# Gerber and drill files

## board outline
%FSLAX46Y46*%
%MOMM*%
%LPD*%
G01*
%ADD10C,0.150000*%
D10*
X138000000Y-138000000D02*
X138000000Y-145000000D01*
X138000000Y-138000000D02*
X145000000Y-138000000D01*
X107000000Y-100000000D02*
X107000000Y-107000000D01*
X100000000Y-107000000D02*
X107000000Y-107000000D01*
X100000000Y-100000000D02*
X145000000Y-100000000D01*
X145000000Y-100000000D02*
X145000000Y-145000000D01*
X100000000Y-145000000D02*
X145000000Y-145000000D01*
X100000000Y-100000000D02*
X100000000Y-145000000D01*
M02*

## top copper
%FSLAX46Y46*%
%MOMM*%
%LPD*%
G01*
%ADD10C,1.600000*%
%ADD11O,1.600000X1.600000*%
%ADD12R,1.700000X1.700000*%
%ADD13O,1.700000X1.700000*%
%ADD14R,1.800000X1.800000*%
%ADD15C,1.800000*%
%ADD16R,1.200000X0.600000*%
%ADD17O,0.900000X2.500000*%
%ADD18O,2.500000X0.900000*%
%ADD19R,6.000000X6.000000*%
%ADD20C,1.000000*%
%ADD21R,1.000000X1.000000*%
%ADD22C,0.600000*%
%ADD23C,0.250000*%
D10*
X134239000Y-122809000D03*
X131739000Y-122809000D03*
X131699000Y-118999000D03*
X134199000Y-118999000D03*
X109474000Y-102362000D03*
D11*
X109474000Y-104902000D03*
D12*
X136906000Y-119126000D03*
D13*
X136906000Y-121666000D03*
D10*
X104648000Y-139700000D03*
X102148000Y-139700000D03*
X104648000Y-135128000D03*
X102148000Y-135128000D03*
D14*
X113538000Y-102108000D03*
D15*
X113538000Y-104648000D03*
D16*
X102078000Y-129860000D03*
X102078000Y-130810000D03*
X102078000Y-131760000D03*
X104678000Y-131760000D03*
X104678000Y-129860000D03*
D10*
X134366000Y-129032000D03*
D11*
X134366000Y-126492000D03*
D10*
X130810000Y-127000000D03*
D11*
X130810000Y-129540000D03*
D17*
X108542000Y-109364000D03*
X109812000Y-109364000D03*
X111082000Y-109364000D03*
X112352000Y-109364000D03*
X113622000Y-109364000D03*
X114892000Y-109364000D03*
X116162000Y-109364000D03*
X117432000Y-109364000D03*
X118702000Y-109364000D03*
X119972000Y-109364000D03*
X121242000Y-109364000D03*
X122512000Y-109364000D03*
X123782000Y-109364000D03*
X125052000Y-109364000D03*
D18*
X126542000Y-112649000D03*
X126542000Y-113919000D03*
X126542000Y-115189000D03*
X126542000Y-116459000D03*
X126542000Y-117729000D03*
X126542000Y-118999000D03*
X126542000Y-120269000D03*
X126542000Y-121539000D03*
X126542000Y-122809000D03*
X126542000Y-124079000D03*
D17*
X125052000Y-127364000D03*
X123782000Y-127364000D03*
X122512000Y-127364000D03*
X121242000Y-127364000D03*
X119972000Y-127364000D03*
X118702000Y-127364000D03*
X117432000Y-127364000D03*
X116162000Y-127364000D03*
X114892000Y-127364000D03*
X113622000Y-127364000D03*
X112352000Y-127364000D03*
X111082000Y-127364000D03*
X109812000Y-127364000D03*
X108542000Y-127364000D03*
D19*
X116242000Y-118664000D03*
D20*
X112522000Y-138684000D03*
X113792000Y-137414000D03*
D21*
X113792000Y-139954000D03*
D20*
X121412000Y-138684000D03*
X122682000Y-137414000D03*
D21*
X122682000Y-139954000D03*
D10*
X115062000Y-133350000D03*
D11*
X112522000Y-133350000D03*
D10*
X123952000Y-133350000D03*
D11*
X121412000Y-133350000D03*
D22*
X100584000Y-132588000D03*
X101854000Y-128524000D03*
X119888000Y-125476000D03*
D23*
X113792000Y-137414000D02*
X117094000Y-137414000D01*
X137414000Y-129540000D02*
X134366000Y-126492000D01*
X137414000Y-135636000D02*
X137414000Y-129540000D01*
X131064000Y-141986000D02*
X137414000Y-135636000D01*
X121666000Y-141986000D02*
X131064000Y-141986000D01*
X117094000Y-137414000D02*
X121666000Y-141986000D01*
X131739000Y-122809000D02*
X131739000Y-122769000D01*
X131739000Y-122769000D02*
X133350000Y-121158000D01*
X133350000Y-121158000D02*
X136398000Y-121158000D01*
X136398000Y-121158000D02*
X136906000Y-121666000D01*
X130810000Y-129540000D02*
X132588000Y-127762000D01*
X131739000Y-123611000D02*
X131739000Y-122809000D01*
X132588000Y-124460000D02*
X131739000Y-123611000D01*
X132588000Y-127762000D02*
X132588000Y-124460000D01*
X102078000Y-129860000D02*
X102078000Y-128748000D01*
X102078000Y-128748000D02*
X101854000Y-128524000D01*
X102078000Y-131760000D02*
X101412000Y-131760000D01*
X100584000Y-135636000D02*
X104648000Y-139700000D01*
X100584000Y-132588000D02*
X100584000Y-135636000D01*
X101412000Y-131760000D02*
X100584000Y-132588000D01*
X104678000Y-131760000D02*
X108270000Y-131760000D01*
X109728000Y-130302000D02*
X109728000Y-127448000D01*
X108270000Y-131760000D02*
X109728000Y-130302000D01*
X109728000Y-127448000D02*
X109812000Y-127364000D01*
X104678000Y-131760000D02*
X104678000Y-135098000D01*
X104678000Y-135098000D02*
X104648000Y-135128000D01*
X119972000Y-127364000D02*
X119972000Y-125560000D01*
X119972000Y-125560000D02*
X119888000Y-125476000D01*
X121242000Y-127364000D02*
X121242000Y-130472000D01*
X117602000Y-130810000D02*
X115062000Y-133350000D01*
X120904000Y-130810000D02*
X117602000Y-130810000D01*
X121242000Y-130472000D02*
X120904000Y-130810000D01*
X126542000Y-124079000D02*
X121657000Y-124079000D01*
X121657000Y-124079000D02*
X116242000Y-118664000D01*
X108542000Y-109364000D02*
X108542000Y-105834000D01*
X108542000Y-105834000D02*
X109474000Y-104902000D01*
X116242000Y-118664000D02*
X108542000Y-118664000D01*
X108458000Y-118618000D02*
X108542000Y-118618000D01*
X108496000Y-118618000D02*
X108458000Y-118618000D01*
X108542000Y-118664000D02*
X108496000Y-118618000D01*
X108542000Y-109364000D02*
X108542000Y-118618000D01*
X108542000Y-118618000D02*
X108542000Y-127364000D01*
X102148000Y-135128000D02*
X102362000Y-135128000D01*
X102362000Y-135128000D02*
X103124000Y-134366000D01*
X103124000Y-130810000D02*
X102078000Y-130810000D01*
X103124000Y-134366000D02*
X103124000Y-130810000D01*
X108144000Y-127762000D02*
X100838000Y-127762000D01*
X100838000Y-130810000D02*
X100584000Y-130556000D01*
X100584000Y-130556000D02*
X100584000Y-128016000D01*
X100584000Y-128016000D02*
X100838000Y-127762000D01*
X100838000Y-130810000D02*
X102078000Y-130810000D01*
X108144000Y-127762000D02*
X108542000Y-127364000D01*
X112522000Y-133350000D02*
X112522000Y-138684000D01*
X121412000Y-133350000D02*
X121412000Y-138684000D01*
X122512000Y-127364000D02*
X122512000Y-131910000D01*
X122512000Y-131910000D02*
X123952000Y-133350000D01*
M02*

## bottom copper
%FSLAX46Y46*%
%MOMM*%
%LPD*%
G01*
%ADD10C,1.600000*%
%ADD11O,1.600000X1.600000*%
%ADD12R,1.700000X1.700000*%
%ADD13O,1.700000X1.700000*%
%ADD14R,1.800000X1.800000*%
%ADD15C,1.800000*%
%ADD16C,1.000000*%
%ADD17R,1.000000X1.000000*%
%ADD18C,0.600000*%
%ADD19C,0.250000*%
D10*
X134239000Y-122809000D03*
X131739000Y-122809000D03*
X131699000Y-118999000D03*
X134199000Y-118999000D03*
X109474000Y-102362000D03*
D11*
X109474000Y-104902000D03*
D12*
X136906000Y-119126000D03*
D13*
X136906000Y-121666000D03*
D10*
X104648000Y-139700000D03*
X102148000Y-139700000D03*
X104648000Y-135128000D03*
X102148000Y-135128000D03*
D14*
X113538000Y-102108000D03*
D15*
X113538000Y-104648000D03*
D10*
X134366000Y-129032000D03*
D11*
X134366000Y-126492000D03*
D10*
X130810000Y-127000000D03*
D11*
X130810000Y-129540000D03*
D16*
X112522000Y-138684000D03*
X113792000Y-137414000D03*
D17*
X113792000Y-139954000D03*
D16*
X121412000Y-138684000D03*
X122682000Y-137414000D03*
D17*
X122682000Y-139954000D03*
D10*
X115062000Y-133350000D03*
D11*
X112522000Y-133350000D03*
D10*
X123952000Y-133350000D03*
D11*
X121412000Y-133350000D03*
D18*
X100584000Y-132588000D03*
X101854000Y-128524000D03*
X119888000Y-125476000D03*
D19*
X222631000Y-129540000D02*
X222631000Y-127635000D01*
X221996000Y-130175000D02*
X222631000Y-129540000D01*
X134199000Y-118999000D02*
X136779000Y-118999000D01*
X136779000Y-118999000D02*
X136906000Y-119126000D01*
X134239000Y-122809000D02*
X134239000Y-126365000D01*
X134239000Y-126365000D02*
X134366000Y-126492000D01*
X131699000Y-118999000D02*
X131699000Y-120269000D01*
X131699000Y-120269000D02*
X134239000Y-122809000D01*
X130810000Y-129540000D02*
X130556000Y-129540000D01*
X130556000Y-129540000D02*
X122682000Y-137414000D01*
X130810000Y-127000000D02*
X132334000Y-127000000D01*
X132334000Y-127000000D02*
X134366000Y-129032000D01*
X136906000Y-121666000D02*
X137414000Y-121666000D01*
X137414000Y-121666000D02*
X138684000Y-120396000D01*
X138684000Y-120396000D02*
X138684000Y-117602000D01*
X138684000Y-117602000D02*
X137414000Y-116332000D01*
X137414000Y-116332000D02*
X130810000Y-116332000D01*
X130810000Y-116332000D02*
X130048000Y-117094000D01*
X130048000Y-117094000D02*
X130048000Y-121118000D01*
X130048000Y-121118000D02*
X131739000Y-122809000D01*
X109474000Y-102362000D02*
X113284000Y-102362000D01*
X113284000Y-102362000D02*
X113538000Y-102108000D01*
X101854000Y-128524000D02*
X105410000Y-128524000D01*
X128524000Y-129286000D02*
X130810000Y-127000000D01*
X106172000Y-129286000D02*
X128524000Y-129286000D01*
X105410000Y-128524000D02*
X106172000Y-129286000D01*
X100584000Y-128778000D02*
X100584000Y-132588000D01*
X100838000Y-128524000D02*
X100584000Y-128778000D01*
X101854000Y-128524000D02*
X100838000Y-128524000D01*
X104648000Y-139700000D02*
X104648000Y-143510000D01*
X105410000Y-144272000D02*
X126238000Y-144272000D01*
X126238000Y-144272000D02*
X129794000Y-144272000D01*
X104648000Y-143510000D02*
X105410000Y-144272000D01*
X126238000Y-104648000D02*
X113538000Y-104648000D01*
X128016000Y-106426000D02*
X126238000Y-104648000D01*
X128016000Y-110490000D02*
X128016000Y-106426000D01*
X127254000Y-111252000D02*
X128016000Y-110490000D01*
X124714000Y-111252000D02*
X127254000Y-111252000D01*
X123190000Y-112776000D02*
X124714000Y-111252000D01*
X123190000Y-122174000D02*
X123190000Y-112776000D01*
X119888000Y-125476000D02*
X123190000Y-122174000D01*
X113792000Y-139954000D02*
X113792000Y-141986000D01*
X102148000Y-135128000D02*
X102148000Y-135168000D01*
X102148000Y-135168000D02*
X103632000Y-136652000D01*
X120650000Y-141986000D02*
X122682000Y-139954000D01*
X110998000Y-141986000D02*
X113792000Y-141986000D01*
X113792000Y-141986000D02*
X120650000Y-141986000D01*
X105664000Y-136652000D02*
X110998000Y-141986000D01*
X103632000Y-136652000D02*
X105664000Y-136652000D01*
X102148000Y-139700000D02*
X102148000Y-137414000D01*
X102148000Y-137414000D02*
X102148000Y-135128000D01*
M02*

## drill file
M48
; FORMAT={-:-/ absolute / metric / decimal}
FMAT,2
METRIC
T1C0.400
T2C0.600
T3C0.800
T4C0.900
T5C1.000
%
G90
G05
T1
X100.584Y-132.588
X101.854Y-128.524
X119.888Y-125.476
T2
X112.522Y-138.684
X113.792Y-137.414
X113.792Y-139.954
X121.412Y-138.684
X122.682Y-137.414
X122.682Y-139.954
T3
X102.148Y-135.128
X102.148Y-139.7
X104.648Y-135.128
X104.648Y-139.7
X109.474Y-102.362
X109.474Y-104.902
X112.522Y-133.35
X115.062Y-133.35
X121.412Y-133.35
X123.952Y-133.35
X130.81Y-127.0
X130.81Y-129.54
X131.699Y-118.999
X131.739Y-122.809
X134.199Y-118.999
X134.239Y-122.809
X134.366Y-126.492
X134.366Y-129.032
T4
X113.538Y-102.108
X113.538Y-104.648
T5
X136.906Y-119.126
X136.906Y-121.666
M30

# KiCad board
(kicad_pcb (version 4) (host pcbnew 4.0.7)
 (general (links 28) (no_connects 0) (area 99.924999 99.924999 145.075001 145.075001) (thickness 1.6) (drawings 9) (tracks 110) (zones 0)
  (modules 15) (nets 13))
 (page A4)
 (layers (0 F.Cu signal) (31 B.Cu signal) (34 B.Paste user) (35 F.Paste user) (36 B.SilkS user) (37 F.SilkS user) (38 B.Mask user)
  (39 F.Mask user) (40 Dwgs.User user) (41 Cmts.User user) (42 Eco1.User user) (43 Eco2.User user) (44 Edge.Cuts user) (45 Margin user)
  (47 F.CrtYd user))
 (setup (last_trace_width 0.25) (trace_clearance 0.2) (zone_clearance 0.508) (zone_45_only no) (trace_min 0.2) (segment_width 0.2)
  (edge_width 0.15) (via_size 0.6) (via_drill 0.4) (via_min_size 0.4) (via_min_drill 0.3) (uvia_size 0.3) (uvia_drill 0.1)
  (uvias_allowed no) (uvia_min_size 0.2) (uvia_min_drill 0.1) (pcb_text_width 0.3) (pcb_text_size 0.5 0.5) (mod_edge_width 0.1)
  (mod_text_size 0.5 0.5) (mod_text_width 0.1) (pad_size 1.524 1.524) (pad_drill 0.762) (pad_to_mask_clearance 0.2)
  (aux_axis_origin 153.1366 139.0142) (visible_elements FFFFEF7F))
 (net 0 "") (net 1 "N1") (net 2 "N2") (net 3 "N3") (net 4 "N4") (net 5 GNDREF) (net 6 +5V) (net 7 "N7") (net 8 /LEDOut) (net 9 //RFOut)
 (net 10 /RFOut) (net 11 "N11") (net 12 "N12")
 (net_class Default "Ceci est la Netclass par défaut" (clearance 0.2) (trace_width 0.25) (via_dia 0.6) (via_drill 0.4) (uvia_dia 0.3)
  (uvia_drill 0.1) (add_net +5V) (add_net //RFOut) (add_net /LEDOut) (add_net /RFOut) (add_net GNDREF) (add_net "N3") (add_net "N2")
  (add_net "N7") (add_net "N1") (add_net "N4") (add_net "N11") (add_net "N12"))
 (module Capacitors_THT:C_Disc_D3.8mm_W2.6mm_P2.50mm (layer F.Cu) (at 134.239 122.809 180)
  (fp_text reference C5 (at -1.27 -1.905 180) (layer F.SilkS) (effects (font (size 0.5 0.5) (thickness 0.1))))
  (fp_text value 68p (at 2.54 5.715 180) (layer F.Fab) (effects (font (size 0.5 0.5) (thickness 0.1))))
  (pad 1 thru_hole circle (at 0 0 180) (size 1.6 1.6) (drill 0.8) (layers *.Cu *.Mask) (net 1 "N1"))
  (pad 2 thru_hole circle (at 2.5 0 180) (size 1.6 1.6) (drill 0.8) (layers *.Cu *.Mask) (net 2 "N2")))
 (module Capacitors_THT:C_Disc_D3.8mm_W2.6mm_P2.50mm (layer F.Cu) (at 131.699 118.999)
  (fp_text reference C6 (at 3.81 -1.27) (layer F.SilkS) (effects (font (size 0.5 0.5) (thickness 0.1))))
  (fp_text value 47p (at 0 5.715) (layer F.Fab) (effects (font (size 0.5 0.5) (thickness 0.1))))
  (pad 1 thru_hole circle (at 0 0) (size 1.6 1.6) (drill 0.8) (layers *.Cu *.Mask) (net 1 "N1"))
  (pad 2 thru_hole circle (at 2.5 0) (size 1.6 1.6) (drill 0.8) (layers *.Cu *.Mask) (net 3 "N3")))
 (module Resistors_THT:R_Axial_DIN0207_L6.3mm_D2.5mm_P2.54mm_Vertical (layer F.Cu) (at 109.474 102.362 270)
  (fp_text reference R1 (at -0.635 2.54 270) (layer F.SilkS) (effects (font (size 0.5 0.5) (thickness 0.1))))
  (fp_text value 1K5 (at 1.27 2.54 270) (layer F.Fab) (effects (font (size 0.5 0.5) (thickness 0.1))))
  (pad 1 thru_hole circle (at 0 0 270) (size 1.6 1.6) (drill 0.8) (layers *.Cu *.Mask) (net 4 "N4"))
  (pad 2 thru_hole oval (at 2.54 0 270) (size 1.6 1.6) (drill 0.8) (layers *.Cu *.Mask) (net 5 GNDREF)))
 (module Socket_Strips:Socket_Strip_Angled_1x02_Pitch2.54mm (layer B.Cu) (at 136.906 119.126 180)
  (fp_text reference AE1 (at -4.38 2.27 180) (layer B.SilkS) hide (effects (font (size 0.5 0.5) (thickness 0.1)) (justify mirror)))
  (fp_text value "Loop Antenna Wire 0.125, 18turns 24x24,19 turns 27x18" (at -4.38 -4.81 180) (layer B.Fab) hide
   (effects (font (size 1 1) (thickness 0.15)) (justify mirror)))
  (pad 1 thru_hole rect (at 0 0 180) (size 1.7 1.7) (drill 1) (layers *.Cu *.Mask) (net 3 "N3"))
  (pad 2 thru_hole oval (at 0 -2.54 180) (size 1.7 1.7) (drill 1) (layers *.Cu *.Mask) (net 2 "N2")))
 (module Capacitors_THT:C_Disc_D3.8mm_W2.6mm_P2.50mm (layer F.Cu) (at 104.648 139.7 180)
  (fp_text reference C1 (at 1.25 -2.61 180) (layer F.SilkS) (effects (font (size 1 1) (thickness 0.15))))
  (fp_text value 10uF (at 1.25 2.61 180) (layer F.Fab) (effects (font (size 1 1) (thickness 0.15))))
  (pad 1 thru_hole circle (at 0 0 180) (size 1.6 1.6) (drill 0.8) (layers *.Cu *.Mask) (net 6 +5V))
  (pad 2 thru_hole circle (at 2.5 0 180) (size 1.6 1.6) (drill 0.8) (layers *.Cu *.Mask) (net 5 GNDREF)))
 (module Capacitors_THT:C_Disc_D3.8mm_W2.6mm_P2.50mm (layer F.Cu) (at 104.648 135.128 180)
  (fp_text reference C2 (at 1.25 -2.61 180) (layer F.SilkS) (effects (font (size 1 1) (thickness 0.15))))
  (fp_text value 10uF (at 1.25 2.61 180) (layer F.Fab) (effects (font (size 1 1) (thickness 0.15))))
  (pad 1 thru_hole circle (at 0 0 180) (size 1.6 1.6) (drill 0.8) (layers *.Cu *.Mask) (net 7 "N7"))
  (pad 2 thru_hole circle (at 2.5 0 180) (size 1.6 1.6) (drill 0.8) (layers *.Cu *.Mask) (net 5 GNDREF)))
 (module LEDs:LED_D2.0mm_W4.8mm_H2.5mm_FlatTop (layer F.Cu) (at 113.538 102.108 270)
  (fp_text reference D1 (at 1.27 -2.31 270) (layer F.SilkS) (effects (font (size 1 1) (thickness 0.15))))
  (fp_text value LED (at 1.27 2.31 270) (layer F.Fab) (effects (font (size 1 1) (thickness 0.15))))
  (pad 1 thru_hole rect (at 0 0 270) (size 1.8 1.8) (drill 0.9) (layers *.Cu *.Mask) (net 4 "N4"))
  (pad 2 thru_hole circle (at 2.54 0 270) (size 1.8 1.8) (drill 0.9) (layers *.Cu *.Mask) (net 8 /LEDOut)))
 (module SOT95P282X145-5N (layer F.Cu) (at 103.378 130.81)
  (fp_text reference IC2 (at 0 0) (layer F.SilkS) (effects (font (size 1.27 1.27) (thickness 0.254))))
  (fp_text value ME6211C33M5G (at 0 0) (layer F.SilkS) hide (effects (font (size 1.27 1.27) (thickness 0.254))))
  (pad 1 smd rect (at -1.3 -0.95 90) (size 0.6 1.2) (layers F.Cu F.Paste F.Mask) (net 6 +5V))
  (pad 2 smd rect (at -1.3 0 90) (size 0.6 1.2) (layers F.Cu F.Paste F.Mask) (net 5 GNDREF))
  (pad 3 smd rect (at -1.3 0.95 90) (size 0.6 1.2) (layers F.Cu F.Paste F.Mask) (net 6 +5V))
  (pad 4 smd rect (at 1.3 0.95 90) (size 0.6 1.2) (layers F.Cu F.Paste F.Mask) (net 7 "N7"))
  (pad 5 smd rect (at 1.3 -0.95 90) (size 0.6 1.2) (layers F.Cu F.Paste F.Mask)))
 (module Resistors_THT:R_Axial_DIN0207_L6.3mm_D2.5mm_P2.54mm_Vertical (layer F.Cu) (at 134.366 129.032 90)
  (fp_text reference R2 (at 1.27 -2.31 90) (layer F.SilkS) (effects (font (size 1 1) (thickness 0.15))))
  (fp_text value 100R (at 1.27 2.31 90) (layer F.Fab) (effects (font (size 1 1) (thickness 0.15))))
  (pad 1 thru_hole circle (at 0 0 90) (size 1.6 1.6) (drill 0.8) (layers *.Cu *.Mask) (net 6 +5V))
  (pad 2 thru_hole oval (at 2.54 0 90) (size 1.6 1.6) (drill 0.8) (layers *.Cu *.Mask) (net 1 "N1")))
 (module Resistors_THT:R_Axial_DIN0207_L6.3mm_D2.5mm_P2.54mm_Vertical (layer F.Cu) (at 130.81 127 270)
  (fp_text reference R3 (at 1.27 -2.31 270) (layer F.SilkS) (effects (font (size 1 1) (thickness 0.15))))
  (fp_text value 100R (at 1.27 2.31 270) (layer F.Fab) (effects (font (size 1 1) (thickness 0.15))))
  (pad 1 thru_hole circle (at 0 0 270) (size 1.6 1.6) (drill 0.8) (layers *.Cu *.Mask) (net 6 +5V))
  (pad 2 thru_hole oval (at 2.54 0 270) (size 1.6 1.6) (drill 0.8) (layers *.Cu *.Mask) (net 2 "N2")))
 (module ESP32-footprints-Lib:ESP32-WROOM (layer F.Cu) (at 113.792 118.364 270)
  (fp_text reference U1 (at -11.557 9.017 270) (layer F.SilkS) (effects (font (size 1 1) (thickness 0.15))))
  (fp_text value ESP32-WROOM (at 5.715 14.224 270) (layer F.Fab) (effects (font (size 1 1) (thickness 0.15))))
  (pad 38 smd oval (at -9 5.25 270) (size 2.5 0.9) (layers F.Cu F.Paste F.Mask) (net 5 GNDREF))
  (pad 37 smd oval (at -9 3.98 270) (size 2.5 0.9) (layers F.Cu F.Paste F.Mask))
  (pad 36 smd oval (at -9 2.71 270) (size 2.5 0.9) (layers F.Cu F.Paste F.Mask))
  (pad 35 smd oval (at -9 1.44 270) (size 2.5 0.9) (layers F.Cu F.Paste F.Mask))
  (pad 34 smd oval (at -9 0.17 270) (size 2.5 0.9) (layers F.Cu F.Paste F.Mask))
  (pad 33 smd oval (at -9 -1.1 270) (size 2.5 0.9) (layers F.Cu F.Paste F.Mask))
  (pad 32 smd oval (at -9 -2.37 270) (size 2.5 0.9) (layers F.Cu F.Paste F.Mask))
  (pad 31 smd oval (at -9 -3.64 270) (size 2.5 0.9) (layers F.Cu F.Paste F.Mask))
  (pad 30 smd oval (at -9 -4.91 270) (size 2.5 0.9) (layers F.Cu F.Paste F.Mask))
  (pad 29 smd oval (at -9 -6.18 270) (size 2.5 0.9) (layers F.Cu F.Paste F.Mask))
  (pad 28 smd oval (at -9 -7.45 270) (size 2.5 0.9) (layers F.Cu F.Paste F.Mask))
  (pad 27 smd oval (at -9 -8.72 270) (size 2.5 0.9) (layers F.Cu F.Paste F.Mask))
  (pad 26 smd oval (at -9 -9.99 270) (size 2.5 0.9) (layers F.Cu F.Paste F.Mask))
  (pad 25 smd oval (at -9 -11.26 270) (size 2.5 0.9) (layers F.Cu F.Paste F.Mask))
  (pad 24 smd oval (at -5.715 -12.75 270) (size 0.9 2.5) (layers F.Cu F.Paste F.Mask))
  (pad 23 smd oval (at -4.445 -12.75 270) (size 0.9 2.5) (layers F.Cu F.Paste F.Mask))
  (pad 22 smd oval (at -3.175 -12.75 270) (size 0.9 2.5) (layers F.Cu F.Paste F.Mask))
  (pad 21 smd oval (at -1.905 -12.75 270) (size 0.9 2.5) (layers F.Cu F.Paste F.Mask))
  (pad 20 smd oval (at -0.635 -12.75 270) (size 0.9 2.5) (layers F.Cu F.Paste F.Mask))
  (pad 19 smd oval (at 0.635 -12.75 270) (size 0.9 2.5) (layers F.Cu F.Paste F.Mask))
  (pad 18 smd oval (at 1.905 -12.75 270) (size 0.9 2.5) (layers F.Cu F.Paste F.Mask))
  (pad 17 smd oval (at 3.175 -12.75 270) (size 0.9 2.5) (layers F.Cu F.Paste F.Mask))
  (pad 16 smd oval (at 4.445 -12.75 270) (size 0.9 2.5) (layers F.Cu F.Paste F.Mask))
  (pad 15 smd oval (at 5.715 -12.75 270) (size 0.9 2.5) (layers F.Cu F.Paste F.Mask) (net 5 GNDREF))
  (pad 14 smd oval (at 9 -11.26 270) (size 2.5 0.9) (layers F.Cu F.Paste F.Mask))
  (pad 13 smd oval (at 9 -9.99 270) (size 2.5 0.9) (layers F.Cu F.Paste F.Mask))
  (pad 12 smd oval (at 9 -8.72 270) (size 2.5 0.9) (layers F.Cu F.Paste F.Mask) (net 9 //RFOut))
  (pad 11 smd oval (at 9 -7.45 270) (size 2.5 0.9) (layers F.Cu F.Paste F.Mask) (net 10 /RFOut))
  (pad 10 smd oval (at 9 -6.18 270) (size 2.5 0.9) (layers F.Cu F.Paste F.Mask) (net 8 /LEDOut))
  (pad 9 smd oval (at 9 -4.91 270) (size 2.5 0.9) (layers F.Cu F.Paste F.Mask))
  (pad 8 smd oval (at 9 -3.64 270) (size 2.5 0.9) (layers F.Cu F.Paste F.Mask))
  (pad 7 smd oval (at 9 -2.37 270) (size 2.5 0.9) (layers F.Cu F.Paste F.Mask))
  (pad 6 smd oval (at 9 -1.1 270) (size 2.5 0.9) (layers F.Cu F.Paste F.Mask))
  (pad 5 smd oval (at 9 0.17 270) (size 2.5 0.9) (layers F.Cu F.Paste F.Mask))
  (pad 4 smd oval (at 9 1.44 270) (size 2.5 0.9) (layers F.Cu F.Paste F.Mask))
  (pad 3 smd oval (at 9 2.71 270) (size 2.5 0.9) (layers F.Cu F.Paste F.Mask))
  (pad 2 smd oval (at 9 3.98 270) (size 2.5 0.9) (layers F.Cu F.Paste F.Mask) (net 7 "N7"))
  (pad 1 smd oval (at 9 5.25 270) (size 2.5 0.9) (layers F.Cu F.Paste F.Mask) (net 5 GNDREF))
  (pad 39 smd rect (at 0.3 -2.45 270) (size 6 6) (layers F.Cu F.Paste F.Mask) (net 5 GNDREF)))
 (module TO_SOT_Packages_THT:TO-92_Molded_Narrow (layer F.Cu) (at 113.792 139.954 90)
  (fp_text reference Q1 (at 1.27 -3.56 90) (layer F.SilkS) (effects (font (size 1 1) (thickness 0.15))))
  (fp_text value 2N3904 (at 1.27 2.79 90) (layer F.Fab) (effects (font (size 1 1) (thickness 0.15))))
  (pad 2 thru_hole circle (at 1.27 -1.27 180) (size 1 1) (drill 0.6) (layers *.Cu *.Mask) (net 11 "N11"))
  (pad 3 thru_hole circle (at 2.54 0 180) (size 1 1) (drill 0.6) (layers *.Cu *.Mask) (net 1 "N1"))
  (pad 1 thru_hole rect (at 0 0 180) (size 1 1) (drill 0.6) (layers *.Cu *.Mask) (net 5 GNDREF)))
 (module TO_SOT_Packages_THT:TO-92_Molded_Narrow (layer F.Cu) (at 122.682 139.954 90)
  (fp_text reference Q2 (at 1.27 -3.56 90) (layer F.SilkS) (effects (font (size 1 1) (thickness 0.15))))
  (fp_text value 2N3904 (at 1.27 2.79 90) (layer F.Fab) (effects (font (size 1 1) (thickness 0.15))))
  (pad 2 thru_hole circle (at 1.27 -1.27 180) (size 1 1) (drill 0.6) (layers *.Cu *.Mask) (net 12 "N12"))
  (pad 3 thru_hole circle (at 2.54 0 180) (size 1 1) (drill 0.6) (layers *.Cu *.Mask) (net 2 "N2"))
  (pad 1 thru_hole rect (at 0 0 180) (size 1 1) (drill 0.6) (layers *.Cu *.Mask) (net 5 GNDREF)))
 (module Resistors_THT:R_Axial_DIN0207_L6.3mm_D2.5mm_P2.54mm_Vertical (layer F.Cu) (at 115.062 133.35 180)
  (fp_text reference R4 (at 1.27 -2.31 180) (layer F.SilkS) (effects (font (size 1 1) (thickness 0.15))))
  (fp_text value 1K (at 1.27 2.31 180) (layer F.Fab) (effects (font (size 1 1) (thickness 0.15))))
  (pad 1 thru_hole circle (at 0 0 180) (size 1.6 1.6) (drill 0.8) (layers *.Cu *.Mask) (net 10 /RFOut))
  (pad 2 thru_hole oval (at 2.54 0 180) (size 1.6 1.6) (drill 0.8) (layers *.Cu *.Mask) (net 11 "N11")))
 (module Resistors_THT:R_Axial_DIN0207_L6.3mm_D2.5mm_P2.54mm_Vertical (layer F.Cu) (at 123.952 133.35 180)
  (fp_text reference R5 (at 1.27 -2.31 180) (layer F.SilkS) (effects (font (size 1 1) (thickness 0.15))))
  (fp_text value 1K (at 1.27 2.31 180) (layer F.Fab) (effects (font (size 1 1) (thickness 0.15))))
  (pad 1 thru_hole circle (at 0 0 180) (size 1.6 1.6) (drill 0.8) (layers *.Cu *.Mask) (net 9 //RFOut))
  (pad 2 thru_hole oval (at 2.54 0 180) (size 1.6 1.6) (drill 0.8) (layers *.Cu *.Mask) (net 12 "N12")))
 (gr_line (start 138 138) (end 138 145) (angle 90) (layer Edge.Cuts) (width 0.15))
 (gr_line (start 138 138) (end 145 138) (angle 90) (layer Edge.Cuts) (width 0.15))
 (gr_line (start 107 100) (end 107 107) (angle 90) (layer Edge.Cuts) (width 0.15))
 (gr_line (start 100 107) (end 107 107) (angle 90) (layer Edge.Cuts) (width 0.15))
 (gr_line (start 100 100) (end 145 100) (angle 90) (layer Edge.Cuts) (width 0.15))
 (gr_line (start 145 100) (end 145 145) (angle 90) (layer Edge.Cuts) (width 0.15))
 (gr_line (start 100 145) (end 145 145) (angle 90) (layer Edge.Cuts) (width 0.15))
 (gr_line (start 100 100) (end 100 145) (angle 90) (layer Edge.Cuts) (width 0.15))
 (segment (start 222.631 129.54) (end 222.631 127.635) (width 0.25) (layer B.Cu) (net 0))
 (segment (start 221.996 130.175) (end 222.631 129.54) (width 0.25) (layer B.Cu) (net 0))
 (segment (start 134.199 118.999) (end 136.779 118.999) (width 0.25) (layer B.Cu) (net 3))
 (segment (start 136.779 118.999) (end 136.906 119.126) (width 0.25) (layer B.Cu) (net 3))
 (segment (start 113.792 137.414) (end 117.094 137.414) (width 0.25) (layer F.Cu) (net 1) (status 400000))
 (segment (start 137.414 129.54) (end 134.366 126.492) (width 0.25) (layer F.Cu) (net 1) (status 800000))
 (segment (start 137.414 135.636) (end 137.414 129.54) (width 0.25) (layer F.Cu) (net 1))
 (segment (start 131.064 141.986) (end 137.414 135.636) (width 0.25) (layer F.Cu) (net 1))
 (segment (start 121.666 141.986) (end 131.064 141.986) (width 0.25) (layer F.Cu) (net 1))
 (segment (start 117.094 137.414) (end 121.666 141.986) (width 0.25) (layer F.Cu) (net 1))
 (segment (start 134.239 122.809) (end 134.239 126.365) (width 0.25) (layer B.Cu) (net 1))
 (segment (start 134.239 126.365) (end 134.366 126.492) (width 0.25) (layer B.Cu) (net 1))
 (segment (start 131.699 118.999) (end 131.699 120.269) (width 0.25) (layer B.Cu) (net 1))
 (segment (start 131.699 120.269) (end 134.239 122.809) (width 0.25) (layer B.Cu) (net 1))
 (segment (start 131.739 122.809) (end 131.739 122.769) (width 0.25) (layer F.Cu) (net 2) (status C00000))
 (segment (start 131.739 122.769) (end 133.35 121.158) (width 0.25) (layer F.Cu) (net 2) (status 400000))
 (segment (start 133.35 121.158) (end 136.398 121.158) (width 0.25) (layer F.Cu) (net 2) (status 800000))
 (segment (start 136.398 121.158) (end 136.906 121.666) (width 0.25) (layer F.Cu) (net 2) (status C00000))
 (segment (start 130.81 129.54) (end 132.588 127.762) (width 0.25) (layer F.Cu) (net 2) (status 400000))
 (segment (start 131.739 123.611) (end 131.739 122.809) (width 0.25) (layer F.Cu) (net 2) (status 800000))
 (segment (start 132.588 124.46) (end 131.739 123.611) (width 0.25) (layer F.Cu) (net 2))
 (segment (start 132.588 127.762) (end 132.588 124.46) (width 0.25) (layer F.Cu) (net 2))
 (segment (start 130.81 129.54) (end 130.556 129.54) (width 0.25) (layer B.Cu) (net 2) (status C00000))
 (segment (start 130.556 129.54) (end 122.682 137.414) (width 0.25) (layer B.Cu) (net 2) (status C00000))
 (segment (start 130.81 127) (end 132.334 127) (width 0.25) (layer B.Cu) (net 6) (status 400000))
 (segment (start 132.334 127) (end 134.366 129.032) (width 0.25) (layer B.Cu) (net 6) (status 800000))
 (segment (start 136.906 121.666) (end 137.414 121.666) (width 0.25) (layer B.Cu) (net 2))
 (segment (start 137.414 121.666) (end 138.684 120.396) (width 0.25) (layer B.Cu) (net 2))
 (segment (start 138.684 120.396) (end 138.684 117.602) (width 0.25) (layer B.Cu) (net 2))
 (segment (start 138.684 117.602) (end 137.414 116.332) (width 0.25) (layer B.Cu) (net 2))
 (segment (start 137.414 116.332) (end 130.81 116.332) (width 0.25) (layer B.Cu) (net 2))
 (segment (start 130.81 116.332) (end 130.048 117.094) (width 0.25) (layer B.Cu) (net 2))
 (segment (start 130.048 117.094) (end 130.048 121.118) (width 0.25) (layer B.Cu) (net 2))
 (segment (start 130.048 121.118) (end 131.739 122.809) (width 0.25) (layer B.Cu) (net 2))
 (segment (start 109.474 102.362) (end 113.284 102.362) (width 0.25) (layer B.Cu) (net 4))
 (segment (start 113.284 102.362) (end 113.538 102.108) (width 0.25) (layer B.Cu) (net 4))
 (segment (start 101.854 128.524) (end 105.41 128.524) (width 0.25) (layer B.Cu) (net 6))
 (segment (start 128.524 129.286) (end 130.81 127) (width 0.25) (layer B.Cu) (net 6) (status 800000))
 (segment (start 106.172 129.286) (end 128.524 129.286) (width 0.25) (layer B.Cu) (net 6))
 (segment (start 105.41 128.524) (end 106.172 129.286) (width 0.25) (layer B.Cu) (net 6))
 (segment (start 102.078 129.86) (end 102.078 128.748) (width 0.25) (layer F.Cu) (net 6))
 (via (at 100.584 132.588) (size 0.6) (drill 0.4) (layers F.Cu B.Cu) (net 6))
 (segment (start 100.584 128.778) (end 100.584 132.588) (width 0.25) (layer B.Cu) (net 6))
 (segment (start 100.838 128.524) (end 100.584 128.778) (width 0.25) (layer B.Cu) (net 6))
 (segment (start 101.854 128.524) (end 100.838 128.524) (width 0.25) (layer B.Cu) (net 6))
 (via (at 101.854 128.524) (size 0.6) (drill 0.4) (layers F.Cu B.Cu) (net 6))
 (segment (start 102.078 128.748) (end 101.854 128.524) (width 0.25) (layer F.Cu) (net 6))
 (segment (start 102.078 131.76) (end 101.412 131.76) (width 0.25) (layer F.Cu) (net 6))
 (segment (start 100.584 135.636) (end 104.648 139.7) (width 0.25) (layer F.Cu) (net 6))
 (segment (start 100.584 132.588) (end 100.584 135.636) (width 0.25) (layer F.Cu) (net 6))
 (segment (start 101.412 131.76) (end 100.584 132.588) (width 0.25) (layer F.Cu) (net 6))
 (segment (start 104.648 139.7) (end 104.648 143.51) (width 0.25) (layer B.Cu) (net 6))
 (segment (start 105.41 144.272) (end 126.238 144.272) (width 0.25) (layer B.Cu) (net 6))
 (segment (start 126.238 144.272) (end 129.794 144.272) (width 0.25) (layer B.Cu) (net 6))
 (segment (start 104.648 143.51) (end 105.41 144.272) (width 0.25) (layer B.Cu) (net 6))
 (segment (start 104.678 131.76) (end 108.27 131.76) (width 0.25) (layer F.Cu) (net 7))
 (segment (start 109.728 130.302) (end 109.728 127.448) (width 0.25) (layer F.Cu) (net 7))
 (segment (start 108.27 131.76) (end 109.728 130.302) (width 0.25) (layer F.Cu) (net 7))
 (segment (start 109.728 127.448) (end 109.812 127.364) (width 0.25) (layer F.Cu) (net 7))
 (segment (start 104.678 131.76) (end 104.678 135.098) (width 0.25) (layer F.Cu) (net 7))
 (segment (start 104.678 135.098) (end 104.648 135.128) (width 0.25) (layer F.Cu) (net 7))
 (segment (start 119.972 127.364) (end 119.972 125.56) (width 0.25) (layer F.Cu) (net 8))
 (segment (start 126.238 104.648) (end 113.538 104.648) (width 0.25) (layer B.Cu) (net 8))
 (segment (start 128.016 106.426) (end 126.238 104.648) (width 0.25) (layer B.Cu) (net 8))
 (segment (start 128.016 110.49) (end 128.016 106.426) (width 0.25) (layer B.Cu) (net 8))
 (segment (start 127.254 111.252) (end 128.016 110.49) (width 0.25) (layer B.Cu) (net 8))
 (segment (start 124.714 111.252) (end 127.254 111.252) (width 0.25) (layer B.Cu) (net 8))
 (segment (start 123.19 112.776) (end 124.714 111.252) (width 0.25) (layer B.Cu) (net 8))
 (segment (start 123.19 122.174) (end 123.19 112.776) (width 0.25) (layer B.Cu) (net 8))
 (segment (start 119.888 125.476) (end 123.19 122.174) (width 0.25) (layer B.Cu) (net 8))
 (via (at 119.888 125.476) (size 0.6) (drill 0.4) (layers F.Cu B.Cu) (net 8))
 (segment (start 119.972 125.56) (end 119.888 125.476) (width 0.25) (layer F.Cu) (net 8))
 (segment (start 121.242 127.364) (end 121.242 130.472) (width 0.25) (layer F.Cu) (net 10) (status 400000))
 (segment (start 117.602 130.81) (end 115.062 133.35) (width 0.25) (layer F.Cu) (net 10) (status 800000))
 (segment (start 120.904 130.81) (end 117.602 130.81) (width 0.25) (layer F.Cu) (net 10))
 (segment (start 121.242 130.472) (end 120.904 130.81) (width 0.25) (layer F.Cu) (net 10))
 (segment (start 113.792 139.954) (end 113.792 141.986) (width 0.25) (layer B.Cu) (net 5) (status 400000))
 (segment (start 102.148 135.128) (end 102.148 135.168) (width 0.25) (layer B.Cu) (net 5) (status C00000))
 (segment (start 102.148 135.168) (end 103.632 136.652) (width 0.25) (layer B.Cu) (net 5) (status 400000))
 (segment (start 120.65 141.986) (end 122.682 139.954) (width 0.25) (layer B.Cu) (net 5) (status 800000))
 (segment (start 110.998 141.986) (end 113.792 141.986) (width 0.25) (layer B.Cu) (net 5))
 (segment (start 113.792 141.986) (end 120.65 141.986) (width 0.25) (layer B.Cu) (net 5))
 (segment (start 105.664 136.652) (end 110.998 141.986) (width 0.25) (layer B.Cu) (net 5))
 (segment (start 103.632 136.652) (end 105.664 136.652) (width 0.25) (layer B.Cu) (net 5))
 (segment (start 126.542 124.079) (end 121.657 124.079) (width 0.25) (layer F.Cu) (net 5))
 (segment (start 121.657 124.079) (end 116.242 118.664) (width 0.25) (layer F.Cu) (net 5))
 (segment (start 108.542 109.364) (end 108.542 105.834) (width 0.25) (layer F.Cu) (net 5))
 (segment (start 108.542 105.834) (end 109.474 104.902) (width 0.25) (layer F.Cu) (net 5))
 (segment (start 116.242 118.664) (end 108.542 118.664) (width 0.25) (layer F.Cu) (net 5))
 (segment (start 108.458 118.618) (end 108.542 118.618) (width 0.25) (layer F.Cu) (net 5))
 (segment (start 108.496 118.618) (end 108.458 118.618) (width 0.25) (layer F.Cu) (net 5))
 (segment (start 108.542 118.664) (end 108.496 118.618) (width 0.25) (layer F.Cu) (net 5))
 (segment (start 108.542 109.364) (end 108.542 118.618) (width 0.25) (layer F.Cu) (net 5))
 (segment (start 108.542 118.618) (end 108.542 127.364) (width 0.25) (layer F.Cu) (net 5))
 (segment (start 102.148 135.128) (end 102.362 135.128) (width 0.25) (layer F.Cu) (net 5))
 (segment (start 102.362 135.128) (end 103.124 134.366) (width 0.25) (layer F.Cu) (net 5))
 (segment (start 103.124 130.81) (end 102.078 130.81) (width 0.25) (layer F.Cu) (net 5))
 (segment (start 103.124 134.366) (end 103.124 130.81) (width 0.25) (layer F.Cu) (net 5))
 (segment (start 108.144 127.762) (end 100.838 127.762) (width 0.25) (layer F.Cu) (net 5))
 (segment (start 100.838 130.81) (end 100.584 130.556) (width 0.25) (layer F.Cu) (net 5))
 (segment (start 100.584 130.556) (end 100.584 128.016) (width 0.25) (layer F.Cu) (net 5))
 (segment (start 100.584 128.016) (end 100.838 127.762) (width 0.25) (layer F.Cu) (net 5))
 (segment (start 100.838 130.81) (end 102.078 130.81) (width 0.25) (layer F.Cu) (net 5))
 (segment (start 108.144 127.762) (end 108.542 127.364) (width 0.25) (layer F.Cu) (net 5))
 (segment (start 102.148 139.7) (end 102.148 137.414) (width 0.25) (layer B.Cu) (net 5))
 (segment (start 102.148 137.414) (end 102.148 135.128) (width 0.25) (layer B.Cu) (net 5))
 (segment (start 112.522 133.35) (end 112.522 138.684) (width 0.25) (layer F.Cu) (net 11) (status C00000))
 (segment (start 121.412 133.35) (end 121.412 138.684) (width 0.25) (layer F.Cu) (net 12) (status C00000))
 (segment (start 122.512 127.364) (end 122.512 131.91) (width 0.25) (layer F.Cu) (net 9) (status 400000))
 (segment (start 122.512 131.91) (end 123.952 133.35) (width 0.25) (layer F.Cu) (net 9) (status 800000)))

